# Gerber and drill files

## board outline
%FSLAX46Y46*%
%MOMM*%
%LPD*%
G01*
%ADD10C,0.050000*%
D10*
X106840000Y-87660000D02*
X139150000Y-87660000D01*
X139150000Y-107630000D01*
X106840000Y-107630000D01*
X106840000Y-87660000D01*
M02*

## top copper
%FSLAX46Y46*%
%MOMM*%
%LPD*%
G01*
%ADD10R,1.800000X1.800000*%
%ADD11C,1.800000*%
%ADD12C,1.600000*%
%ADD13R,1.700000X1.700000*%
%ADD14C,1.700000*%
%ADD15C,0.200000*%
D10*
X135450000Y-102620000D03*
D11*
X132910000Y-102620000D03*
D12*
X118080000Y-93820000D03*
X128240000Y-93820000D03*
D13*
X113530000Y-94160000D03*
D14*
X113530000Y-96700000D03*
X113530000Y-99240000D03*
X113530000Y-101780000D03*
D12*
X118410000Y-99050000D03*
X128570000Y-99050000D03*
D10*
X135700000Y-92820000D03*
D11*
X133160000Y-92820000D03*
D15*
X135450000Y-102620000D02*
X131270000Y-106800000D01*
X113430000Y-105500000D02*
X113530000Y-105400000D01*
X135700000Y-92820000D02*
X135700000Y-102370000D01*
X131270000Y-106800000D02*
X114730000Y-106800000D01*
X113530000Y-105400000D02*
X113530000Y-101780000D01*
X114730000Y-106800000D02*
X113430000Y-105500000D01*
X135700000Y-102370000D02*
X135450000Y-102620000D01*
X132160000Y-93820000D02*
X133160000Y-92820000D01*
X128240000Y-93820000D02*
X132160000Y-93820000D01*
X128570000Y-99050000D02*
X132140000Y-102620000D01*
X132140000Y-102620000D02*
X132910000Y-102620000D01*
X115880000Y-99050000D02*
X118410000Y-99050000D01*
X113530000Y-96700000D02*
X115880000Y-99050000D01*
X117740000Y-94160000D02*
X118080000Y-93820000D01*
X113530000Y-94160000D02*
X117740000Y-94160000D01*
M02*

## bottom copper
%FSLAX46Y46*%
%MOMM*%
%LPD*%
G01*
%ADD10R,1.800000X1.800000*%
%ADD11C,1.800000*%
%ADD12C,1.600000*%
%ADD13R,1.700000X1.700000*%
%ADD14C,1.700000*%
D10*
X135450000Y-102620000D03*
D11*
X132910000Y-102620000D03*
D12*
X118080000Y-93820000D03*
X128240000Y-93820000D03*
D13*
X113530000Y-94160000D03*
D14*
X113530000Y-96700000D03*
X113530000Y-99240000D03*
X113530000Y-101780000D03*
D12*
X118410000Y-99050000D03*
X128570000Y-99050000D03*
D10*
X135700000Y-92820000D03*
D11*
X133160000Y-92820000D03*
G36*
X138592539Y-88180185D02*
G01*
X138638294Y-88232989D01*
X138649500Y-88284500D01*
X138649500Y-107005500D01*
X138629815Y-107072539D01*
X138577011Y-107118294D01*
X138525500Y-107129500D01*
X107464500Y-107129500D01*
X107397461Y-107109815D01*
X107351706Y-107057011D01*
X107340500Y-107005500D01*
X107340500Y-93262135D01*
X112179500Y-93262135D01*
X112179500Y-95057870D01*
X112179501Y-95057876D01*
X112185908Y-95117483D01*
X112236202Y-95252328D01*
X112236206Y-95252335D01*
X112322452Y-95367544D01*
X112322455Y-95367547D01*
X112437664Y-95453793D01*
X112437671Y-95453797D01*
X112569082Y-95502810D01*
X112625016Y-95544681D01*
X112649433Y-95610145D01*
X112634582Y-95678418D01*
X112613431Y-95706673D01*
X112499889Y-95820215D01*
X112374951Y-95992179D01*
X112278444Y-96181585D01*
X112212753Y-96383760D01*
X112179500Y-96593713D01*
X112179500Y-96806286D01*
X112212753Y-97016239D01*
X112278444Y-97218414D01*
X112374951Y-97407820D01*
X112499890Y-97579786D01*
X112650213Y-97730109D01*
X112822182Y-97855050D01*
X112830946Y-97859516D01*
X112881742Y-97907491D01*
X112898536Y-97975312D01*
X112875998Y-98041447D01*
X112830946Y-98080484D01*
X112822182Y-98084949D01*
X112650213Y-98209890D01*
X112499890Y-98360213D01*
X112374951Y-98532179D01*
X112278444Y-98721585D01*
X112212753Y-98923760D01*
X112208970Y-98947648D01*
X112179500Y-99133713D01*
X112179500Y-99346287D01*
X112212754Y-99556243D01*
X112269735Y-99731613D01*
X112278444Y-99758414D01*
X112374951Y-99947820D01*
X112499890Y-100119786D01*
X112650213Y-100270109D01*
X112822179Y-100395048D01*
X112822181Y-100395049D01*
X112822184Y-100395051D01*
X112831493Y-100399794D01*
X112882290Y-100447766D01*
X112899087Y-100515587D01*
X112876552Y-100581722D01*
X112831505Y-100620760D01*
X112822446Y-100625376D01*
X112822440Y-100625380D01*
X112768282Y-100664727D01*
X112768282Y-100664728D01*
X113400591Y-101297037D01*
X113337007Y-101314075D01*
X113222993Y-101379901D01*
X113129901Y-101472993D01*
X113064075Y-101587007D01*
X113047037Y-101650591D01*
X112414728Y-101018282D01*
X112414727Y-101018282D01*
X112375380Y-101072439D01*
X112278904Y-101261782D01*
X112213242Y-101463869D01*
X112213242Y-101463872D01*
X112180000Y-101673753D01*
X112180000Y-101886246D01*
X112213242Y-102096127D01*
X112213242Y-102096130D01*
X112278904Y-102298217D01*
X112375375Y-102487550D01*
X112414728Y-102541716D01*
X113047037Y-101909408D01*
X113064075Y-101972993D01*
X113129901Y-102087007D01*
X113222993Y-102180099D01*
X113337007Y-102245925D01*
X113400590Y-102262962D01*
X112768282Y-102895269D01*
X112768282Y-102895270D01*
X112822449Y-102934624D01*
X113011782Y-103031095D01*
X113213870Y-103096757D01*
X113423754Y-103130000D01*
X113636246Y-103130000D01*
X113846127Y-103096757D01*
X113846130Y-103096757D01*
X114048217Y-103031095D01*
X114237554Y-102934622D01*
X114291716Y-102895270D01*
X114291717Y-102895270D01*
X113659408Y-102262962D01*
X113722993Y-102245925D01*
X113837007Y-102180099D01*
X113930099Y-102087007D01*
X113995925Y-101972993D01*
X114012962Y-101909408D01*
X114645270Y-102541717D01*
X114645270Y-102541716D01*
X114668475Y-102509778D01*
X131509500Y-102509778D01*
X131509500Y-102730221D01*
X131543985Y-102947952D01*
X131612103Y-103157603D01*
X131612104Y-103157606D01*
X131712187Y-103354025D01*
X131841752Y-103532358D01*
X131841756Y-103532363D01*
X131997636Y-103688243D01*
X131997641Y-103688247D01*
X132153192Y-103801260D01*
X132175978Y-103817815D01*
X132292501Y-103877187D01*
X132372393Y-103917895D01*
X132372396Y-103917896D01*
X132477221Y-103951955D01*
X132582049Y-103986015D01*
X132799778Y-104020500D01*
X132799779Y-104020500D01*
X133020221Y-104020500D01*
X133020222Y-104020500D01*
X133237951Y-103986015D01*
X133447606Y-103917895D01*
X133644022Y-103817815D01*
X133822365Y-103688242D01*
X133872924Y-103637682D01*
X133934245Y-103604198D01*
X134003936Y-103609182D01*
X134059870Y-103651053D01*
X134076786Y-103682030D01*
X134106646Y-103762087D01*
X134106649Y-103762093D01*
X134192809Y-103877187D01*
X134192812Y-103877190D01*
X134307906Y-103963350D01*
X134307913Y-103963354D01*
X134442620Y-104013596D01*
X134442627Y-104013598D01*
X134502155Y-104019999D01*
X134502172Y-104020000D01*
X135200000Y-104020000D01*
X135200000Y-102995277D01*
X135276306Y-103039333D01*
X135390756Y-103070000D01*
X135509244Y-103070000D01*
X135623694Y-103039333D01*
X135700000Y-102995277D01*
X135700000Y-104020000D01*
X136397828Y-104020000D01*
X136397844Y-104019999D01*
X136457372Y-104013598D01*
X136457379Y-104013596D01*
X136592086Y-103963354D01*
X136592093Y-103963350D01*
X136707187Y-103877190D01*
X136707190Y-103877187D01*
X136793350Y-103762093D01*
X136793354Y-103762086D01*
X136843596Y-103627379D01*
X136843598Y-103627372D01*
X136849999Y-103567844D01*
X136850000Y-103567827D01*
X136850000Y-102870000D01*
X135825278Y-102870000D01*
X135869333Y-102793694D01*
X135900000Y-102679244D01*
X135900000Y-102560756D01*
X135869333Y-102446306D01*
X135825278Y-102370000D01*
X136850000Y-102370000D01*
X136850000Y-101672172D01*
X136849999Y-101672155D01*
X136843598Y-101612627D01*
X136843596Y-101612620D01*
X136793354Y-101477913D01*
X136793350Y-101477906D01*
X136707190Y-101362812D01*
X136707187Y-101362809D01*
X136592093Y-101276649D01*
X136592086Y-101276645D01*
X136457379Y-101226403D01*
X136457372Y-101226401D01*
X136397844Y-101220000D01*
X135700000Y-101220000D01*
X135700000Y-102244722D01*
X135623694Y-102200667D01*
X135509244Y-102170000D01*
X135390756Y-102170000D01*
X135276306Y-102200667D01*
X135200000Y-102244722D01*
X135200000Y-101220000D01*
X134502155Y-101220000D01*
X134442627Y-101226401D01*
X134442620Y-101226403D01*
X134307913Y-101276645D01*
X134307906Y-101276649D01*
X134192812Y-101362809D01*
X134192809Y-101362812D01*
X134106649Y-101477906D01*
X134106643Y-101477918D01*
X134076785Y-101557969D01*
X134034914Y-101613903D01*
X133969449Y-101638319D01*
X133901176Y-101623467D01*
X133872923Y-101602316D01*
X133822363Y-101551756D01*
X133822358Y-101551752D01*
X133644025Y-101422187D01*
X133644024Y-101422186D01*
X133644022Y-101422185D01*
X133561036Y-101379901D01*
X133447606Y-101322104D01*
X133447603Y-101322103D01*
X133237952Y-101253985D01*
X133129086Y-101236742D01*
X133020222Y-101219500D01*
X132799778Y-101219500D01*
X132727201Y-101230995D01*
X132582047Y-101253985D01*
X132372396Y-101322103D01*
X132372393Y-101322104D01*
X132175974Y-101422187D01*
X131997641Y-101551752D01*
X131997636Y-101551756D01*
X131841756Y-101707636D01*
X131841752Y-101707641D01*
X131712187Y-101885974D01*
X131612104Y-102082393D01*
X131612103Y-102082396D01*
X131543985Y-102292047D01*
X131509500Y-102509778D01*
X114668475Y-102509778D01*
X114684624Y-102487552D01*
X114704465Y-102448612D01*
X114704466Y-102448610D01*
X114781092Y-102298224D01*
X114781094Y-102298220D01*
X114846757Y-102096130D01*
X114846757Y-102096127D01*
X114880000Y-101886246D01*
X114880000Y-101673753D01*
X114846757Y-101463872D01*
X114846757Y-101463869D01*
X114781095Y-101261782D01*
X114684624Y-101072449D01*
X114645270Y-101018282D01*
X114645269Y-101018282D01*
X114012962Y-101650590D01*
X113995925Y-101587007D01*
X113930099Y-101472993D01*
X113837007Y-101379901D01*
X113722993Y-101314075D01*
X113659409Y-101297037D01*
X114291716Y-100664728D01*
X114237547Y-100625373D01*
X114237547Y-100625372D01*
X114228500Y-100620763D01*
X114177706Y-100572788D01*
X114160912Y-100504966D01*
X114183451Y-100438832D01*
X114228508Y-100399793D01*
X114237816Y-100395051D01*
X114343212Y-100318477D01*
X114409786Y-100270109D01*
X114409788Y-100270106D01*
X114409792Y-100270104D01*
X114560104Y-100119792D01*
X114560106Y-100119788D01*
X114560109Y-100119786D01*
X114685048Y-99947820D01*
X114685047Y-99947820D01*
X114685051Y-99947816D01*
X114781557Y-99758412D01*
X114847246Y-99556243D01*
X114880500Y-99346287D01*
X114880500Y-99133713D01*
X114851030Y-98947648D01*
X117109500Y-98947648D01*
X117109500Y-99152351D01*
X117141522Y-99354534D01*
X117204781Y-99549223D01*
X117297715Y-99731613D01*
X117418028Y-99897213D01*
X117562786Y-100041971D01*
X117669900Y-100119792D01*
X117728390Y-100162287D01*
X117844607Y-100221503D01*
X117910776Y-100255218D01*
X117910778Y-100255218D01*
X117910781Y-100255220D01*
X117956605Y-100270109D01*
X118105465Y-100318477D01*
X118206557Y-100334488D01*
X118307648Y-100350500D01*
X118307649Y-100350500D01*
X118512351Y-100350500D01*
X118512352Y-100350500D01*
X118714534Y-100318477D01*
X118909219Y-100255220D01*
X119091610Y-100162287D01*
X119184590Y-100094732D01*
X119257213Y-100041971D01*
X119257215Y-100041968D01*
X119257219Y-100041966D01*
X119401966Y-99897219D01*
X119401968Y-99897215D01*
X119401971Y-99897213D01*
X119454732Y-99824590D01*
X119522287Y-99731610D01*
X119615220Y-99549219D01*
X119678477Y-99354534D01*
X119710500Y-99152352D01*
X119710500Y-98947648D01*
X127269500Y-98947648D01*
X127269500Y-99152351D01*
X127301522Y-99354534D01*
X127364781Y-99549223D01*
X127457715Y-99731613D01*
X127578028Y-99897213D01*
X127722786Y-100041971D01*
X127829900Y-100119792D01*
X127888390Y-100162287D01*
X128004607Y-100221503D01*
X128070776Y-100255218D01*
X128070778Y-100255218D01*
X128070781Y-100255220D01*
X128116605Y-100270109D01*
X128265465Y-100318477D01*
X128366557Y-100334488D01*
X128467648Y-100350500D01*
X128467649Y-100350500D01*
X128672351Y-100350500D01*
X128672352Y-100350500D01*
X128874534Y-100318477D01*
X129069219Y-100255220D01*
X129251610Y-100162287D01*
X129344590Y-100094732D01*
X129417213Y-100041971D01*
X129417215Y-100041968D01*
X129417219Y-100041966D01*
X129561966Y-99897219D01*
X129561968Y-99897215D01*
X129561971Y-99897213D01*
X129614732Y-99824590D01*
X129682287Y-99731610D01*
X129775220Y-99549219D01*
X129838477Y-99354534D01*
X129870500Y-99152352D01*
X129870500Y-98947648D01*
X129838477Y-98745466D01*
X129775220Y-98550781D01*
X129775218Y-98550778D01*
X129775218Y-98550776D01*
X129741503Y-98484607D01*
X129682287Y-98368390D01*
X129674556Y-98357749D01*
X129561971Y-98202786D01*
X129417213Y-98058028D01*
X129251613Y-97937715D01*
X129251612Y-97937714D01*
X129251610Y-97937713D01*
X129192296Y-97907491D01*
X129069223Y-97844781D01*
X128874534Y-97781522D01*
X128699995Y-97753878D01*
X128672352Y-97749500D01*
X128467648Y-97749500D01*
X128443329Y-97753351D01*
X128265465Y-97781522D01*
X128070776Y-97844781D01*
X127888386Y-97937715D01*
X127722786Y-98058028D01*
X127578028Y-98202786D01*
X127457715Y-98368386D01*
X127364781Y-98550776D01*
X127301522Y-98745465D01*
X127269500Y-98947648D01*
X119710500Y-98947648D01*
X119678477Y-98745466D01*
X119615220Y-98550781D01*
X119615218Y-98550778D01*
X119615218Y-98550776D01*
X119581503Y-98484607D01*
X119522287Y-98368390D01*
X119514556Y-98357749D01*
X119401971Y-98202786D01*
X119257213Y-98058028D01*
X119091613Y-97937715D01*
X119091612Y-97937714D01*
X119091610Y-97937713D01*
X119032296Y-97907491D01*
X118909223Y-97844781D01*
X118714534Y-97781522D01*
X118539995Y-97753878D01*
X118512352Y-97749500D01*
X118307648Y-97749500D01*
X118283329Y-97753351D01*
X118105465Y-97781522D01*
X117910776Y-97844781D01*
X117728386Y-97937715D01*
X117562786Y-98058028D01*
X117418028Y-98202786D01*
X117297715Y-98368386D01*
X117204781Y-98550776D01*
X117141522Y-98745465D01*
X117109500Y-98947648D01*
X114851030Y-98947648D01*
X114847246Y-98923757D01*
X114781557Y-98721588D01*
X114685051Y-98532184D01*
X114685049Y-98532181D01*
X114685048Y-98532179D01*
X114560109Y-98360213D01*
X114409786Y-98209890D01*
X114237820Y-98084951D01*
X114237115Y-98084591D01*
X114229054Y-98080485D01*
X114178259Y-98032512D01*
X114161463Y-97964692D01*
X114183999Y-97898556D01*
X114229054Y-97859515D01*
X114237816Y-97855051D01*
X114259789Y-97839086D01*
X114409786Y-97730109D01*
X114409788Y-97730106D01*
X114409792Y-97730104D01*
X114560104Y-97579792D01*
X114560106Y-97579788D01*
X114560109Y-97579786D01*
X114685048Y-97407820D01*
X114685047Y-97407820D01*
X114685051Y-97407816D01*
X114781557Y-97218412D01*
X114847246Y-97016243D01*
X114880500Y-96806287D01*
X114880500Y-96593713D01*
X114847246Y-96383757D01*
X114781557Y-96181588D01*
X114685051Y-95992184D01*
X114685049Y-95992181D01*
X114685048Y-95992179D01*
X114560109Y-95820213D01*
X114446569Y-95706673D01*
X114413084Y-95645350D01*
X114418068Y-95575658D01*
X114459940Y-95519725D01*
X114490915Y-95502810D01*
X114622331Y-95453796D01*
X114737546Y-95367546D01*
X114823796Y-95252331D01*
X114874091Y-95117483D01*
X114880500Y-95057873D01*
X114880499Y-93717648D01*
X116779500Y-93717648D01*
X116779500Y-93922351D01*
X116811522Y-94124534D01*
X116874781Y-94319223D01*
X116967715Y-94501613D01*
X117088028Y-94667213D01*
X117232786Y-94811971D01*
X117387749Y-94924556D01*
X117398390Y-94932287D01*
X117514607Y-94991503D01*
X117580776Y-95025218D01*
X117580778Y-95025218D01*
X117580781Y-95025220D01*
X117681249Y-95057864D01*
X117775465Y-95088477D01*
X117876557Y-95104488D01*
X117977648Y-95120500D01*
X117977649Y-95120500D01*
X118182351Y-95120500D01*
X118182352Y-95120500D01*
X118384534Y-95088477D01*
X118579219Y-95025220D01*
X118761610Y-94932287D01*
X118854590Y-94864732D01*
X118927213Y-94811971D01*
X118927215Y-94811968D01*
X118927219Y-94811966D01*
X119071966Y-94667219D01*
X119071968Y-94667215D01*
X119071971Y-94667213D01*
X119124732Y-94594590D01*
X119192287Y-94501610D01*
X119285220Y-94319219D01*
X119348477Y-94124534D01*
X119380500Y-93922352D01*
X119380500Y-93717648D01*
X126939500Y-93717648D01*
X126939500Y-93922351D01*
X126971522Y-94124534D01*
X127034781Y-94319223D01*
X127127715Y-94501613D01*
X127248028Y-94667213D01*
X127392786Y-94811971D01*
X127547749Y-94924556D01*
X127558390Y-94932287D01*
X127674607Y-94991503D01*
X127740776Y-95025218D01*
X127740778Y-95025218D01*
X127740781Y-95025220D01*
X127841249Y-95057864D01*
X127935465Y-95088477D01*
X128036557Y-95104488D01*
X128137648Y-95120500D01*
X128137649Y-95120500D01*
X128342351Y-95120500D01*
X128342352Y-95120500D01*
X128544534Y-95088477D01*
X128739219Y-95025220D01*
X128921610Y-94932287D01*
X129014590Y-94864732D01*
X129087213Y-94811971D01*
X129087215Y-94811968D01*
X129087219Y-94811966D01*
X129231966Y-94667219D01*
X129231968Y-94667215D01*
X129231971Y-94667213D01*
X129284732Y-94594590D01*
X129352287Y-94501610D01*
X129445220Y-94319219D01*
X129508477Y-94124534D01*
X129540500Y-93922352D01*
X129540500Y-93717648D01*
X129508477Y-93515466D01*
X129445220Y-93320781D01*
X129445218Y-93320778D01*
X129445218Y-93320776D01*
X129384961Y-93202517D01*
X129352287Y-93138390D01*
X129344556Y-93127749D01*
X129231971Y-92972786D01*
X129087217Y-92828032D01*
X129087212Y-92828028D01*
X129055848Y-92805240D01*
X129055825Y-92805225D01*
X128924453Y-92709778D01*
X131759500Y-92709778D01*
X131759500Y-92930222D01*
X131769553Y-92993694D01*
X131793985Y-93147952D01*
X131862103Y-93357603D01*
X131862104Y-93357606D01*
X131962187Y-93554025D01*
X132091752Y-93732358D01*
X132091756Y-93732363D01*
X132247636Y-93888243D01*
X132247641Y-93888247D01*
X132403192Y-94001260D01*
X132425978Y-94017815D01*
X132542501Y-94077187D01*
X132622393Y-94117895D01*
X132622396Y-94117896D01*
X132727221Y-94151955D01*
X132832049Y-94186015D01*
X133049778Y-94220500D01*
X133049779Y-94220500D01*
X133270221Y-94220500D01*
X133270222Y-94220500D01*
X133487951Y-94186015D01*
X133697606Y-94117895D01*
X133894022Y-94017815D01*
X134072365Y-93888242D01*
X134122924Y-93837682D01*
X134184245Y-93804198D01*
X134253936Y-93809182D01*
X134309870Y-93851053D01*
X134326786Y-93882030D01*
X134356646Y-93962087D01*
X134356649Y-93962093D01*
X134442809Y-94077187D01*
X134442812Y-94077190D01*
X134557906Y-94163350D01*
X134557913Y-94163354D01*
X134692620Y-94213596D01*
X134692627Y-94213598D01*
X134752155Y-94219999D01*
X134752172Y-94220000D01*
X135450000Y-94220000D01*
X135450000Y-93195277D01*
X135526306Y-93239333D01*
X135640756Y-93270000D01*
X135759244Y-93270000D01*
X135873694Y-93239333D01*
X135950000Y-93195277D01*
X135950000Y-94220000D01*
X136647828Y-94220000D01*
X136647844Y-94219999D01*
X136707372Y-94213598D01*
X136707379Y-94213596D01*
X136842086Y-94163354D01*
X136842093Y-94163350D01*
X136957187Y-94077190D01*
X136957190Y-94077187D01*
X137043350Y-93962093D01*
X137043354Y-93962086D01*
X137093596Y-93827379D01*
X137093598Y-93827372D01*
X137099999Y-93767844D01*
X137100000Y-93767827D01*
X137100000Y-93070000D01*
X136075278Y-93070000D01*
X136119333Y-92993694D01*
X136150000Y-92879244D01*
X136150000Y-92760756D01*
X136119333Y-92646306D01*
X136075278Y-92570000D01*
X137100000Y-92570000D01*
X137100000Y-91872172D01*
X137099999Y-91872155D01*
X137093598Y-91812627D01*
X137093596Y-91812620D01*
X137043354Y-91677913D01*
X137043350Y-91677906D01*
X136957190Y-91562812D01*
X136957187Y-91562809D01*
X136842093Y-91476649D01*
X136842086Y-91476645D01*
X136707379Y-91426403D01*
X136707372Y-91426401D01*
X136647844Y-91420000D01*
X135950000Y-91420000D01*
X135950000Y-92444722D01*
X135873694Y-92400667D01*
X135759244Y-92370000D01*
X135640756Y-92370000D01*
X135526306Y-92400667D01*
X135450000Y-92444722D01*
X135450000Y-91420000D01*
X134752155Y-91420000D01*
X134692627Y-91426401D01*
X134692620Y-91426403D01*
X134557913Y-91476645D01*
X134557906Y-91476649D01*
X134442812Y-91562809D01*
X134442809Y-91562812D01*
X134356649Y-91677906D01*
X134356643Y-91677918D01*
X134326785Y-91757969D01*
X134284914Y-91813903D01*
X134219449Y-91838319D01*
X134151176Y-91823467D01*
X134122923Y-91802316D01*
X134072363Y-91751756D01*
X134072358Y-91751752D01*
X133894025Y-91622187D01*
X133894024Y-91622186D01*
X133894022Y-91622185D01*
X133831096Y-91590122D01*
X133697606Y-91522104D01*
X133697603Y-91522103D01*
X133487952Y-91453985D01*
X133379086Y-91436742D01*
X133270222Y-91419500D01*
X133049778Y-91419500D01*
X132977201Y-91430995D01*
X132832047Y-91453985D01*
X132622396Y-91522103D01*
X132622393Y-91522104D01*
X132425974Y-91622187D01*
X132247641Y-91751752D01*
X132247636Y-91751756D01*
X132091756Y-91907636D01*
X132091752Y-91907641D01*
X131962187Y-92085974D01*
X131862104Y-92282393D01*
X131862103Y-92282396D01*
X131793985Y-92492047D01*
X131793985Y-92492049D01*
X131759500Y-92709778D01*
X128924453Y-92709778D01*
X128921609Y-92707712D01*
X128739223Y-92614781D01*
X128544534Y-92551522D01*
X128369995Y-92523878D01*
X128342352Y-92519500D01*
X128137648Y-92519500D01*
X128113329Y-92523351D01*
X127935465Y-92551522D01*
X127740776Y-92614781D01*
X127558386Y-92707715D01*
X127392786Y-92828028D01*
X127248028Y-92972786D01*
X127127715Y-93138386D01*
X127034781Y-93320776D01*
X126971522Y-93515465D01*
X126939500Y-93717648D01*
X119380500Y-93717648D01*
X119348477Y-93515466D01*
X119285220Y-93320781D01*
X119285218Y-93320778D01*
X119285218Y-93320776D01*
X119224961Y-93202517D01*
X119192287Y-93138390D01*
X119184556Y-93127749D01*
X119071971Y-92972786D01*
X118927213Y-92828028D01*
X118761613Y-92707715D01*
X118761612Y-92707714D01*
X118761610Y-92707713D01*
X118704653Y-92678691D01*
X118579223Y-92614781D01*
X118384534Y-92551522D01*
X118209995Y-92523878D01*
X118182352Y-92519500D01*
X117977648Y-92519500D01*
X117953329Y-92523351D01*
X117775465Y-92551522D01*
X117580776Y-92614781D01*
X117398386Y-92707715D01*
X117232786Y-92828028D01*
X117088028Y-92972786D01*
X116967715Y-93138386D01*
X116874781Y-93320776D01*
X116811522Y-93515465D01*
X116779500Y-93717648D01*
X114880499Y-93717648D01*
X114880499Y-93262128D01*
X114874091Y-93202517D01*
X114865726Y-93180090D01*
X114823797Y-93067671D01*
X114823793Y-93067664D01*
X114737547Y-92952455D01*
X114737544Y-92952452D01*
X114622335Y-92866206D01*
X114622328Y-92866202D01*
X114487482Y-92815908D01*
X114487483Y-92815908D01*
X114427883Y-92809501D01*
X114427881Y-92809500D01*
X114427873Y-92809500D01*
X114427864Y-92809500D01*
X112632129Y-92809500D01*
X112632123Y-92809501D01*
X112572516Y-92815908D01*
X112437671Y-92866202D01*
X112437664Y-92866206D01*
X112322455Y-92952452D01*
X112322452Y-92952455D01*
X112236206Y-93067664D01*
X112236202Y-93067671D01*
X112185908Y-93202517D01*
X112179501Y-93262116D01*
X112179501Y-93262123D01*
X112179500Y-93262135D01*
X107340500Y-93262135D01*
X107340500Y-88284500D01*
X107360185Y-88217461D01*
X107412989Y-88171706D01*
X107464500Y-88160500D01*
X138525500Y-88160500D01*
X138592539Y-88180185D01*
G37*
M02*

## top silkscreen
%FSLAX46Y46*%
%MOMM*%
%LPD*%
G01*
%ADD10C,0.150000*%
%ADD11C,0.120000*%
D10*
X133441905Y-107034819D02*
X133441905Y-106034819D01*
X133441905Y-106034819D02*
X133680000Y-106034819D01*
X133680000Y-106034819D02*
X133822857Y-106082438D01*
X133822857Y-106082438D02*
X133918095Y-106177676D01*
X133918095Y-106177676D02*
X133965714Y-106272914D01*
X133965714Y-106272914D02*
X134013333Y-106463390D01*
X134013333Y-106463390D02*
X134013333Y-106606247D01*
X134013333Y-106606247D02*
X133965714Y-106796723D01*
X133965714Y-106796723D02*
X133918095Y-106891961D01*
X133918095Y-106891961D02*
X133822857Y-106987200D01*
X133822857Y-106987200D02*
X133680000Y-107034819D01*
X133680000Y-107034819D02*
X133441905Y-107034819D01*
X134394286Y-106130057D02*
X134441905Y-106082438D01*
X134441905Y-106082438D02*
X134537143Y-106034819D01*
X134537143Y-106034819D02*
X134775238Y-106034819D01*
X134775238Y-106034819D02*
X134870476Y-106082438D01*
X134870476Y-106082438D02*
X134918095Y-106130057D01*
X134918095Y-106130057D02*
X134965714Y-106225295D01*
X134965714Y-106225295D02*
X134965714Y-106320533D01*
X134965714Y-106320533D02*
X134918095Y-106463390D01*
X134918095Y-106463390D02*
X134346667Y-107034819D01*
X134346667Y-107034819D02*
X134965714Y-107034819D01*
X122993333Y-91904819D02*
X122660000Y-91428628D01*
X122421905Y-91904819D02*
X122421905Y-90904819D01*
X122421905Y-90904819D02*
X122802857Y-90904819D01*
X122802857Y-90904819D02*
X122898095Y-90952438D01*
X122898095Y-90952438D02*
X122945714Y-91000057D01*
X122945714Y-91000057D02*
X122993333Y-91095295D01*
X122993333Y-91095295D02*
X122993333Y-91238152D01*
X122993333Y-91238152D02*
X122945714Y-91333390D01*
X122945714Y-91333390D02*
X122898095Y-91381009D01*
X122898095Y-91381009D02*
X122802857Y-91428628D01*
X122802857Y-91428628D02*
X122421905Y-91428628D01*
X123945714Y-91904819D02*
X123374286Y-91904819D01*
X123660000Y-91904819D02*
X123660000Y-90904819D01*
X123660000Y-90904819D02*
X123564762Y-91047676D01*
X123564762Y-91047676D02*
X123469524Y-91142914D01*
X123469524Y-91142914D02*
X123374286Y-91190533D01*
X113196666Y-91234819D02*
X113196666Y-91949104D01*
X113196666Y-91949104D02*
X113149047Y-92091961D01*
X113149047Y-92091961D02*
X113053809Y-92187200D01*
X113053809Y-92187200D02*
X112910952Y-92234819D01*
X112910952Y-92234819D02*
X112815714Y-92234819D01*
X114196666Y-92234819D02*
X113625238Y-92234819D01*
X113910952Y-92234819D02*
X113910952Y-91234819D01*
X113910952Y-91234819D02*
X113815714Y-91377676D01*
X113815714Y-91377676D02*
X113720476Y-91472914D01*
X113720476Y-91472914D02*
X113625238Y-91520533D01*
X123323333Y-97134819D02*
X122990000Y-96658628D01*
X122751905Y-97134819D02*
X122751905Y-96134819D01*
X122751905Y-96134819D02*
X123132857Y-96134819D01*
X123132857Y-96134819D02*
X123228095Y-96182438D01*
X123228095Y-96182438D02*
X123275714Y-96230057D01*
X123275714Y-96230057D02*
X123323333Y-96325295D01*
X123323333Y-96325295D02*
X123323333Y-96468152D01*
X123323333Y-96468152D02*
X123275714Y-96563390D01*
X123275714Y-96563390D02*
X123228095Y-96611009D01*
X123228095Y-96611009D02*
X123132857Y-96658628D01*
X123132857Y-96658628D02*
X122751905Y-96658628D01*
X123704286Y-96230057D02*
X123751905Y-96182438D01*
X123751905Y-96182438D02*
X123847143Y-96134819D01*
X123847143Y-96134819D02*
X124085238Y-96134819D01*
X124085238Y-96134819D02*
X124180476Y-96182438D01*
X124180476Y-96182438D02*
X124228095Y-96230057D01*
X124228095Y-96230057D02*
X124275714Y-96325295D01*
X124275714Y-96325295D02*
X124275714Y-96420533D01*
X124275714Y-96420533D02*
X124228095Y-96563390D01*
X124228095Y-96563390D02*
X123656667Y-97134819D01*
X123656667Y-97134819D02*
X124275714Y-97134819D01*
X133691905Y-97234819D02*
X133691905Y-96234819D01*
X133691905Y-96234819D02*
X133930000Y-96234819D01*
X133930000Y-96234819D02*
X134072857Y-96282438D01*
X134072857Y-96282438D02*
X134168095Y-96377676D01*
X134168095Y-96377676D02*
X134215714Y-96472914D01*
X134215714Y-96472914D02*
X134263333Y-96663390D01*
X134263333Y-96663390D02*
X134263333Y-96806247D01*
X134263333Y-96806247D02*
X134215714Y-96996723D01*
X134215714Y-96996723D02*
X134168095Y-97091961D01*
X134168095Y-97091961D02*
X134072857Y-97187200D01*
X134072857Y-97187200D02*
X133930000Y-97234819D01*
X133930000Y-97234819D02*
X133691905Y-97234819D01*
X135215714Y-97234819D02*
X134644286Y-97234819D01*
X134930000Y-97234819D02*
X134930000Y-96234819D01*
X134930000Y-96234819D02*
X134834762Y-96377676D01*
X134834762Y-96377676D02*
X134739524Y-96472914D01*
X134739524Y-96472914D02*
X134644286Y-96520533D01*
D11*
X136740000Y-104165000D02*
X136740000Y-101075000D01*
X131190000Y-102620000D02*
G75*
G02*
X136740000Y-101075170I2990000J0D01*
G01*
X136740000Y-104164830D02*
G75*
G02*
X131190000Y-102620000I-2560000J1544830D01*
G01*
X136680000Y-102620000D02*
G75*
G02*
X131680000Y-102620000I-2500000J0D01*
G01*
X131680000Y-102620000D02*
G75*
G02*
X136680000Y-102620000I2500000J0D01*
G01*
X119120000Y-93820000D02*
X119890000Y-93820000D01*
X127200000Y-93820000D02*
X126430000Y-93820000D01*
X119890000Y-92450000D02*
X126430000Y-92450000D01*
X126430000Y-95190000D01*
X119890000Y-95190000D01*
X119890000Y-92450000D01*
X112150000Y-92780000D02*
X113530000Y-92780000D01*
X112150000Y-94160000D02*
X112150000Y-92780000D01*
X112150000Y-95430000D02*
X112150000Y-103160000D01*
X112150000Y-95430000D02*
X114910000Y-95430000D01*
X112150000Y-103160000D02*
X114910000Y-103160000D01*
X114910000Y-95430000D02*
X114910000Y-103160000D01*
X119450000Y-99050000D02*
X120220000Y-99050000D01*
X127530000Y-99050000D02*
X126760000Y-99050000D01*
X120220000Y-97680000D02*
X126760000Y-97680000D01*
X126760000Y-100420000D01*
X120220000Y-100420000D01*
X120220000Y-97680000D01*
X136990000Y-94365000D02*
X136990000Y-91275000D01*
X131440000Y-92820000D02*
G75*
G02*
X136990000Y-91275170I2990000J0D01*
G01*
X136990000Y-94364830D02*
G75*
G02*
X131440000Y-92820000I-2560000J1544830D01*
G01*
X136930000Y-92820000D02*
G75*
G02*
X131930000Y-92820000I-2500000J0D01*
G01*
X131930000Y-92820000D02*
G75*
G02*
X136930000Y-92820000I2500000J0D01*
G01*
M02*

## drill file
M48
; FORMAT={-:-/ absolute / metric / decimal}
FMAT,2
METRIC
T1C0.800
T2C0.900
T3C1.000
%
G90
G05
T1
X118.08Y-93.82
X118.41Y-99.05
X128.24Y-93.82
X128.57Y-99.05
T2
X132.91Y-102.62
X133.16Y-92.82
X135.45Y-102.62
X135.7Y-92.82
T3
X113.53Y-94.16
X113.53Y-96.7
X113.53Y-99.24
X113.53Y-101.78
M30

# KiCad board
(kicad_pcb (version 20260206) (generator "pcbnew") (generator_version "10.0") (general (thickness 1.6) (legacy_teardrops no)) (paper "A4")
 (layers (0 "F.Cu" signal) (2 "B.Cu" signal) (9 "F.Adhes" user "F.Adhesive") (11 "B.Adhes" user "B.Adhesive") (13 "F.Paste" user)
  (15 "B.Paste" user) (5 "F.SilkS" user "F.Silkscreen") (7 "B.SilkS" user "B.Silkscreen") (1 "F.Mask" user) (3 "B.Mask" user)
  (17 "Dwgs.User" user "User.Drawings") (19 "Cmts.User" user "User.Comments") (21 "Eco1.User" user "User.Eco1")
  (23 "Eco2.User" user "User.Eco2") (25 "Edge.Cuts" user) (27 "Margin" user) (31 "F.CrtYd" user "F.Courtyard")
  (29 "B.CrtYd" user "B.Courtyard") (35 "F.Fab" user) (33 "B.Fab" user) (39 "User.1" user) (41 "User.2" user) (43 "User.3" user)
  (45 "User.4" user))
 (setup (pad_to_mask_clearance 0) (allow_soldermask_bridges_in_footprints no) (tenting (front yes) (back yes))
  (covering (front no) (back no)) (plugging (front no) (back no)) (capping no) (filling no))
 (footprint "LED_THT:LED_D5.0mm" (layer "F.Cu") (at 135.45 102.62 180)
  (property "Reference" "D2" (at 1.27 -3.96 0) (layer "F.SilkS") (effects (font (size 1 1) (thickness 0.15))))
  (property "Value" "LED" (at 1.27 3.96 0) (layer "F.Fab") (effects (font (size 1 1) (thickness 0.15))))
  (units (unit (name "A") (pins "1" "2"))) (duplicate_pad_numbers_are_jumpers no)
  (fp_line (start -1.29 -1.545) (end -1.29 1.545) (stroke (width 0.12) (type solid)) (layer "F.SilkS"))
  (fp_arc (start 4.26 0) (mid 2.071779 2.880495) (end -1.29 1.54483) (stroke (width 0.12) (type solid)) (layer "F.SilkS"))
  (fp_arc (start -1.29 -1.54483) (mid 2.071779 -2.880495) (end 4.26 0) (stroke (width 0.12) (type solid)) (layer "F.SilkS"))
  (fp_circle (center 1.27 0) (end 3.77 0) (stroke (width 0.12) (type solid)) (fill no) (layer "F.SilkS"))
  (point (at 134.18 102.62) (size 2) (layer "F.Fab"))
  (pad "1" thru_hole rect (at 0 0 180) (size 1.8 1.8) (drill 0.9) (layers "*.Cu" "*.Mask") (remove_unused_layers no) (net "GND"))
  (pad "2" thru_hole circle (at 2.54 0 180) (size 1.8 1.8) (drill 0.9) (layers "*.Cu" "*.Mask") (remove_unused_layers no) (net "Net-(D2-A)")))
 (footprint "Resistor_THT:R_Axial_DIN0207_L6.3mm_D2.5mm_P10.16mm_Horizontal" (layer "F.Cu") (at 118.08 93.82)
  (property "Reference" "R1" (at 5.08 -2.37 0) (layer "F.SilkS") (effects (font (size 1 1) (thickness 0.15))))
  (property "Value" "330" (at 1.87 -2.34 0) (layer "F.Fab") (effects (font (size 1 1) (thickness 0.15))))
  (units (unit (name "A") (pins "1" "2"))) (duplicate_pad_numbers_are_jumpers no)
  (fp_line (start 1.04 0) (end 1.81 0) (stroke (width 0.12) (type solid)) (layer "F.SilkS"))
  (fp_line (start 9.12 0) (end 8.35 0) (stroke (width 0.12) (type solid)) (layer "F.SilkS"))
  (fp_rect (start 1.81 -1.37) (end 8.35 1.37) (stroke (width 0.12) (type solid)) (fill no) (layer "F.SilkS"))
  (pad "1" thru_hole circle (at 0 0) (size 1.6 1.6) (drill 0.8) (layers "*.Cu" "*.Mask") (remove_unused_layers no) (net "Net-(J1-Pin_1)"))
  (pad "2" thru_hole circle (at 10.16 0) (size 1.6 1.6) (drill 0.8) (layers "*.Cu" "*.Mask") (remove_unused_layers no) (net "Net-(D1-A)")))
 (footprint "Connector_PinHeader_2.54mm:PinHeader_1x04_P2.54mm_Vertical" (layer "F.Cu") (at 113.53 94.16)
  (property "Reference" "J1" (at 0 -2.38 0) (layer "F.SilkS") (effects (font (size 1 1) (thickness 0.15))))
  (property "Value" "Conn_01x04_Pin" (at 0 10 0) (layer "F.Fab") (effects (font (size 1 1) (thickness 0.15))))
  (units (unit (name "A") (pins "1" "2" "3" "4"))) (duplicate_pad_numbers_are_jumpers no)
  (fp_line (start -1.38 -1.38) (end 0 -1.38) (stroke (width 0.12) (type solid)) (layer "F.SilkS"))
  (fp_line (start -1.38 0) (end -1.38 -1.38) (stroke (width 0.12) (type solid)) (layer "F.SilkS"))
  (fp_line (start -1.38 1.27) (end -1.38 9) (stroke (width 0.12) (type solid)) (layer "F.SilkS"))
  (fp_line (start -1.38 1.27) (end 1.38 1.27) (stroke (width 0.12) (type solid)) (layer "F.SilkS"))
  (fp_line (start -1.38 9) (end 1.38 9) (stroke (width 0.12) (type solid)) (layer "F.SilkS"))
  (fp_line (start 1.38 1.27) (end 1.38 9) (stroke (width 0.12) (type solid)) (layer "F.SilkS"))
  (pad "1" thru_hole rect (at 0 0) (size 1.7 1.7) (drill 1) (layers "*.Cu" "*.Mask") (remove_unused_layers no) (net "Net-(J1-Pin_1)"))
  (pad "2" thru_hole circle (at 0 2.54) (size 1.7 1.7) (drill 1) (layers "*.Cu" "*.Mask") (remove_unused_layers no) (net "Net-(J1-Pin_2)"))
  (pad "3" thru_hole circle (at 0 5.08) (size 1.7 1.7) (drill 1) (layers "*.Cu" "*.Mask") (remove_unused_layers no)
   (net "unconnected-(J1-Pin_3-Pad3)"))
  (pad "4" thru_hole circle (at 0 7.62) (size 1.7 1.7) (drill 1) (layers "*.Cu" "*.Mask") (remove_unused_layers no) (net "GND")))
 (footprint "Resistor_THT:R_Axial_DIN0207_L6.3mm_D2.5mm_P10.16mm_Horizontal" (layer "F.Cu") (at 118.41 99.05)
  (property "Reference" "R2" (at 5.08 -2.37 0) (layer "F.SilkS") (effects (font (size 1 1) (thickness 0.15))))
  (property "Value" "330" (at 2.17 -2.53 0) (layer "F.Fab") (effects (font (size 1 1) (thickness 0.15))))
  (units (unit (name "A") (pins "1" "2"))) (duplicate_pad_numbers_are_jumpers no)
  (fp_line (start 1.04 0) (end 1.81 0) (stroke (width 0.12) (type solid)) (layer "F.SilkS"))
  (fp_line (start 9.12 0) (end 8.35 0) (stroke (width 0.12) (type solid)) (layer "F.SilkS"))
  (fp_rect (start 1.81 -1.37) (end 8.35 1.37) (stroke (width 0.12) (type solid)) (fill no) (layer "F.SilkS"))
  (pad "1" thru_hole circle (at 0 0) (size 1.6 1.6) (drill 0.8) (layers "*.Cu" "*.Mask") (remove_unused_layers no) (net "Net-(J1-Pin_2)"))
  (pad "2" thru_hole circle (at 10.16 0) (size 1.6 1.6) (drill 0.8) (layers "*.Cu" "*.Mask") (remove_unused_layers no) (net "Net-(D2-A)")))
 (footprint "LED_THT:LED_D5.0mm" (layer "F.Cu") (at 135.7 92.82 180)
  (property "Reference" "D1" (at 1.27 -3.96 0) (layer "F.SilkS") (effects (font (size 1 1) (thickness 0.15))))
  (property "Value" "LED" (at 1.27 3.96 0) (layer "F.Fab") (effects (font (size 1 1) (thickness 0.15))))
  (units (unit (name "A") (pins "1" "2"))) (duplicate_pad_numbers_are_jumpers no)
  (fp_line (start -1.29 -1.545) (end -1.29 1.545) (stroke (width 0.12) (type solid)) (layer "F.SilkS"))
  (fp_arc (start 4.26 0) (mid 2.071779 2.880495) (end -1.29 1.54483) (stroke (width 0.12) (type solid)) (layer "F.SilkS"))
  (fp_arc (start -1.29 -1.54483) (mid 2.071779 -2.880495) (end 4.26 0) (stroke (width 0.12) (type solid)) (layer "F.SilkS"))
  (fp_circle (center 1.27 0) (end 3.77 0) (stroke (width 0.12) (type solid)) (fill no) (layer "F.SilkS"))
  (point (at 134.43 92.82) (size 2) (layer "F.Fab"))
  (pad "1" thru_hole rect (at 0 0 180) (size 1.8 1.8) (drill 0.9) (layers "*.Cu" "*.Mask") (remove_unused_layers no) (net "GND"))
  (pad "2" thru_hole circle (at 2.54 0 180) (size 1.8 1.8) (drill 0.9) (layers "*.Cu" "*.Mask") (remove_unused_layers no) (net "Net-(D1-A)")))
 (gr_rect (start 106.84 87.66) (end 139.15 107.63) (stroke (width 0.05) (type default)) (fill no) (layer "Edge.Cuts"))
 (segment (start 135.45 102.62) (end 131.27 106.8) (width 0.2) (layer "F.Cu") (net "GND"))
 (segment (start 113.43 105.5) (end 113.53 105.4) (width 0.2) (layer "F.Cu") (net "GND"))
 (segment (start 135.7 92.82) (end 135.7 102.37) (width 0.2) (layer "F.Cu") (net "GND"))
 (segment (start 131.27 106.8) (end 114.73 106.8) (width 0.2) (layer "F.Cu") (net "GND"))
 (segment (start 113.53 105.4) (end 113.53 101.78) (width 0.2) (layer "F.Cu") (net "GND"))
 (segment (start 114.73 106.8) (end 113.43 105.5) (width 0.2) (layer "F.Cu") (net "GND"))
 (segment (start 135.7 102.37) (end 135.45 102.62) (width 0.2) (layer "F.Cu") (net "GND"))
 (segment (start 132.16 93.82) (end 133.16 92.82) (width 0.2) (layer "F.Cu") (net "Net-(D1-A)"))
 (segment (start 128.24 93.82) (end 132.16 93.82) (width 0.2) (layer "F.Cu") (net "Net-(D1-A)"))
 (segment (start 128.57 99.05) (end 132.14 102.62) (width 0.2) (layer "F.Cu") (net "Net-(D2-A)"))
 (segment (start 132.14 102.62) (end 132.91 102.62) (width 0.2) (layer "F.Cu") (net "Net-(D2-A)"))
 (segment (start 115.88 99.05) (end 118.41 99.05) (width 0.2) (layer "F.Cu") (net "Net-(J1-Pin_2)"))
 (segment (start 113.53 96.7) (end 115.88 99.05) (width 0.2) (layer "F.Cu") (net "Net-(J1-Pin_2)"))
 (segment (start 117.74 94.16) (end 118.08 93.82) (width 0.2) (layer "F.Cu") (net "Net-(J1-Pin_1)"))
 (segment (start 113.53 94.16) (end 117.74 94.16) (width 0.2) (layer "F.Cu") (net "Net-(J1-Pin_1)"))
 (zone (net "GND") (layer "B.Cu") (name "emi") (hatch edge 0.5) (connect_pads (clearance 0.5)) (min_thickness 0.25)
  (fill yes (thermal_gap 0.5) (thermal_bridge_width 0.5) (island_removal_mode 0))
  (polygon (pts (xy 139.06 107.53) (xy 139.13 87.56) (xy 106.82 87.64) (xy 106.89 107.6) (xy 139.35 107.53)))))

